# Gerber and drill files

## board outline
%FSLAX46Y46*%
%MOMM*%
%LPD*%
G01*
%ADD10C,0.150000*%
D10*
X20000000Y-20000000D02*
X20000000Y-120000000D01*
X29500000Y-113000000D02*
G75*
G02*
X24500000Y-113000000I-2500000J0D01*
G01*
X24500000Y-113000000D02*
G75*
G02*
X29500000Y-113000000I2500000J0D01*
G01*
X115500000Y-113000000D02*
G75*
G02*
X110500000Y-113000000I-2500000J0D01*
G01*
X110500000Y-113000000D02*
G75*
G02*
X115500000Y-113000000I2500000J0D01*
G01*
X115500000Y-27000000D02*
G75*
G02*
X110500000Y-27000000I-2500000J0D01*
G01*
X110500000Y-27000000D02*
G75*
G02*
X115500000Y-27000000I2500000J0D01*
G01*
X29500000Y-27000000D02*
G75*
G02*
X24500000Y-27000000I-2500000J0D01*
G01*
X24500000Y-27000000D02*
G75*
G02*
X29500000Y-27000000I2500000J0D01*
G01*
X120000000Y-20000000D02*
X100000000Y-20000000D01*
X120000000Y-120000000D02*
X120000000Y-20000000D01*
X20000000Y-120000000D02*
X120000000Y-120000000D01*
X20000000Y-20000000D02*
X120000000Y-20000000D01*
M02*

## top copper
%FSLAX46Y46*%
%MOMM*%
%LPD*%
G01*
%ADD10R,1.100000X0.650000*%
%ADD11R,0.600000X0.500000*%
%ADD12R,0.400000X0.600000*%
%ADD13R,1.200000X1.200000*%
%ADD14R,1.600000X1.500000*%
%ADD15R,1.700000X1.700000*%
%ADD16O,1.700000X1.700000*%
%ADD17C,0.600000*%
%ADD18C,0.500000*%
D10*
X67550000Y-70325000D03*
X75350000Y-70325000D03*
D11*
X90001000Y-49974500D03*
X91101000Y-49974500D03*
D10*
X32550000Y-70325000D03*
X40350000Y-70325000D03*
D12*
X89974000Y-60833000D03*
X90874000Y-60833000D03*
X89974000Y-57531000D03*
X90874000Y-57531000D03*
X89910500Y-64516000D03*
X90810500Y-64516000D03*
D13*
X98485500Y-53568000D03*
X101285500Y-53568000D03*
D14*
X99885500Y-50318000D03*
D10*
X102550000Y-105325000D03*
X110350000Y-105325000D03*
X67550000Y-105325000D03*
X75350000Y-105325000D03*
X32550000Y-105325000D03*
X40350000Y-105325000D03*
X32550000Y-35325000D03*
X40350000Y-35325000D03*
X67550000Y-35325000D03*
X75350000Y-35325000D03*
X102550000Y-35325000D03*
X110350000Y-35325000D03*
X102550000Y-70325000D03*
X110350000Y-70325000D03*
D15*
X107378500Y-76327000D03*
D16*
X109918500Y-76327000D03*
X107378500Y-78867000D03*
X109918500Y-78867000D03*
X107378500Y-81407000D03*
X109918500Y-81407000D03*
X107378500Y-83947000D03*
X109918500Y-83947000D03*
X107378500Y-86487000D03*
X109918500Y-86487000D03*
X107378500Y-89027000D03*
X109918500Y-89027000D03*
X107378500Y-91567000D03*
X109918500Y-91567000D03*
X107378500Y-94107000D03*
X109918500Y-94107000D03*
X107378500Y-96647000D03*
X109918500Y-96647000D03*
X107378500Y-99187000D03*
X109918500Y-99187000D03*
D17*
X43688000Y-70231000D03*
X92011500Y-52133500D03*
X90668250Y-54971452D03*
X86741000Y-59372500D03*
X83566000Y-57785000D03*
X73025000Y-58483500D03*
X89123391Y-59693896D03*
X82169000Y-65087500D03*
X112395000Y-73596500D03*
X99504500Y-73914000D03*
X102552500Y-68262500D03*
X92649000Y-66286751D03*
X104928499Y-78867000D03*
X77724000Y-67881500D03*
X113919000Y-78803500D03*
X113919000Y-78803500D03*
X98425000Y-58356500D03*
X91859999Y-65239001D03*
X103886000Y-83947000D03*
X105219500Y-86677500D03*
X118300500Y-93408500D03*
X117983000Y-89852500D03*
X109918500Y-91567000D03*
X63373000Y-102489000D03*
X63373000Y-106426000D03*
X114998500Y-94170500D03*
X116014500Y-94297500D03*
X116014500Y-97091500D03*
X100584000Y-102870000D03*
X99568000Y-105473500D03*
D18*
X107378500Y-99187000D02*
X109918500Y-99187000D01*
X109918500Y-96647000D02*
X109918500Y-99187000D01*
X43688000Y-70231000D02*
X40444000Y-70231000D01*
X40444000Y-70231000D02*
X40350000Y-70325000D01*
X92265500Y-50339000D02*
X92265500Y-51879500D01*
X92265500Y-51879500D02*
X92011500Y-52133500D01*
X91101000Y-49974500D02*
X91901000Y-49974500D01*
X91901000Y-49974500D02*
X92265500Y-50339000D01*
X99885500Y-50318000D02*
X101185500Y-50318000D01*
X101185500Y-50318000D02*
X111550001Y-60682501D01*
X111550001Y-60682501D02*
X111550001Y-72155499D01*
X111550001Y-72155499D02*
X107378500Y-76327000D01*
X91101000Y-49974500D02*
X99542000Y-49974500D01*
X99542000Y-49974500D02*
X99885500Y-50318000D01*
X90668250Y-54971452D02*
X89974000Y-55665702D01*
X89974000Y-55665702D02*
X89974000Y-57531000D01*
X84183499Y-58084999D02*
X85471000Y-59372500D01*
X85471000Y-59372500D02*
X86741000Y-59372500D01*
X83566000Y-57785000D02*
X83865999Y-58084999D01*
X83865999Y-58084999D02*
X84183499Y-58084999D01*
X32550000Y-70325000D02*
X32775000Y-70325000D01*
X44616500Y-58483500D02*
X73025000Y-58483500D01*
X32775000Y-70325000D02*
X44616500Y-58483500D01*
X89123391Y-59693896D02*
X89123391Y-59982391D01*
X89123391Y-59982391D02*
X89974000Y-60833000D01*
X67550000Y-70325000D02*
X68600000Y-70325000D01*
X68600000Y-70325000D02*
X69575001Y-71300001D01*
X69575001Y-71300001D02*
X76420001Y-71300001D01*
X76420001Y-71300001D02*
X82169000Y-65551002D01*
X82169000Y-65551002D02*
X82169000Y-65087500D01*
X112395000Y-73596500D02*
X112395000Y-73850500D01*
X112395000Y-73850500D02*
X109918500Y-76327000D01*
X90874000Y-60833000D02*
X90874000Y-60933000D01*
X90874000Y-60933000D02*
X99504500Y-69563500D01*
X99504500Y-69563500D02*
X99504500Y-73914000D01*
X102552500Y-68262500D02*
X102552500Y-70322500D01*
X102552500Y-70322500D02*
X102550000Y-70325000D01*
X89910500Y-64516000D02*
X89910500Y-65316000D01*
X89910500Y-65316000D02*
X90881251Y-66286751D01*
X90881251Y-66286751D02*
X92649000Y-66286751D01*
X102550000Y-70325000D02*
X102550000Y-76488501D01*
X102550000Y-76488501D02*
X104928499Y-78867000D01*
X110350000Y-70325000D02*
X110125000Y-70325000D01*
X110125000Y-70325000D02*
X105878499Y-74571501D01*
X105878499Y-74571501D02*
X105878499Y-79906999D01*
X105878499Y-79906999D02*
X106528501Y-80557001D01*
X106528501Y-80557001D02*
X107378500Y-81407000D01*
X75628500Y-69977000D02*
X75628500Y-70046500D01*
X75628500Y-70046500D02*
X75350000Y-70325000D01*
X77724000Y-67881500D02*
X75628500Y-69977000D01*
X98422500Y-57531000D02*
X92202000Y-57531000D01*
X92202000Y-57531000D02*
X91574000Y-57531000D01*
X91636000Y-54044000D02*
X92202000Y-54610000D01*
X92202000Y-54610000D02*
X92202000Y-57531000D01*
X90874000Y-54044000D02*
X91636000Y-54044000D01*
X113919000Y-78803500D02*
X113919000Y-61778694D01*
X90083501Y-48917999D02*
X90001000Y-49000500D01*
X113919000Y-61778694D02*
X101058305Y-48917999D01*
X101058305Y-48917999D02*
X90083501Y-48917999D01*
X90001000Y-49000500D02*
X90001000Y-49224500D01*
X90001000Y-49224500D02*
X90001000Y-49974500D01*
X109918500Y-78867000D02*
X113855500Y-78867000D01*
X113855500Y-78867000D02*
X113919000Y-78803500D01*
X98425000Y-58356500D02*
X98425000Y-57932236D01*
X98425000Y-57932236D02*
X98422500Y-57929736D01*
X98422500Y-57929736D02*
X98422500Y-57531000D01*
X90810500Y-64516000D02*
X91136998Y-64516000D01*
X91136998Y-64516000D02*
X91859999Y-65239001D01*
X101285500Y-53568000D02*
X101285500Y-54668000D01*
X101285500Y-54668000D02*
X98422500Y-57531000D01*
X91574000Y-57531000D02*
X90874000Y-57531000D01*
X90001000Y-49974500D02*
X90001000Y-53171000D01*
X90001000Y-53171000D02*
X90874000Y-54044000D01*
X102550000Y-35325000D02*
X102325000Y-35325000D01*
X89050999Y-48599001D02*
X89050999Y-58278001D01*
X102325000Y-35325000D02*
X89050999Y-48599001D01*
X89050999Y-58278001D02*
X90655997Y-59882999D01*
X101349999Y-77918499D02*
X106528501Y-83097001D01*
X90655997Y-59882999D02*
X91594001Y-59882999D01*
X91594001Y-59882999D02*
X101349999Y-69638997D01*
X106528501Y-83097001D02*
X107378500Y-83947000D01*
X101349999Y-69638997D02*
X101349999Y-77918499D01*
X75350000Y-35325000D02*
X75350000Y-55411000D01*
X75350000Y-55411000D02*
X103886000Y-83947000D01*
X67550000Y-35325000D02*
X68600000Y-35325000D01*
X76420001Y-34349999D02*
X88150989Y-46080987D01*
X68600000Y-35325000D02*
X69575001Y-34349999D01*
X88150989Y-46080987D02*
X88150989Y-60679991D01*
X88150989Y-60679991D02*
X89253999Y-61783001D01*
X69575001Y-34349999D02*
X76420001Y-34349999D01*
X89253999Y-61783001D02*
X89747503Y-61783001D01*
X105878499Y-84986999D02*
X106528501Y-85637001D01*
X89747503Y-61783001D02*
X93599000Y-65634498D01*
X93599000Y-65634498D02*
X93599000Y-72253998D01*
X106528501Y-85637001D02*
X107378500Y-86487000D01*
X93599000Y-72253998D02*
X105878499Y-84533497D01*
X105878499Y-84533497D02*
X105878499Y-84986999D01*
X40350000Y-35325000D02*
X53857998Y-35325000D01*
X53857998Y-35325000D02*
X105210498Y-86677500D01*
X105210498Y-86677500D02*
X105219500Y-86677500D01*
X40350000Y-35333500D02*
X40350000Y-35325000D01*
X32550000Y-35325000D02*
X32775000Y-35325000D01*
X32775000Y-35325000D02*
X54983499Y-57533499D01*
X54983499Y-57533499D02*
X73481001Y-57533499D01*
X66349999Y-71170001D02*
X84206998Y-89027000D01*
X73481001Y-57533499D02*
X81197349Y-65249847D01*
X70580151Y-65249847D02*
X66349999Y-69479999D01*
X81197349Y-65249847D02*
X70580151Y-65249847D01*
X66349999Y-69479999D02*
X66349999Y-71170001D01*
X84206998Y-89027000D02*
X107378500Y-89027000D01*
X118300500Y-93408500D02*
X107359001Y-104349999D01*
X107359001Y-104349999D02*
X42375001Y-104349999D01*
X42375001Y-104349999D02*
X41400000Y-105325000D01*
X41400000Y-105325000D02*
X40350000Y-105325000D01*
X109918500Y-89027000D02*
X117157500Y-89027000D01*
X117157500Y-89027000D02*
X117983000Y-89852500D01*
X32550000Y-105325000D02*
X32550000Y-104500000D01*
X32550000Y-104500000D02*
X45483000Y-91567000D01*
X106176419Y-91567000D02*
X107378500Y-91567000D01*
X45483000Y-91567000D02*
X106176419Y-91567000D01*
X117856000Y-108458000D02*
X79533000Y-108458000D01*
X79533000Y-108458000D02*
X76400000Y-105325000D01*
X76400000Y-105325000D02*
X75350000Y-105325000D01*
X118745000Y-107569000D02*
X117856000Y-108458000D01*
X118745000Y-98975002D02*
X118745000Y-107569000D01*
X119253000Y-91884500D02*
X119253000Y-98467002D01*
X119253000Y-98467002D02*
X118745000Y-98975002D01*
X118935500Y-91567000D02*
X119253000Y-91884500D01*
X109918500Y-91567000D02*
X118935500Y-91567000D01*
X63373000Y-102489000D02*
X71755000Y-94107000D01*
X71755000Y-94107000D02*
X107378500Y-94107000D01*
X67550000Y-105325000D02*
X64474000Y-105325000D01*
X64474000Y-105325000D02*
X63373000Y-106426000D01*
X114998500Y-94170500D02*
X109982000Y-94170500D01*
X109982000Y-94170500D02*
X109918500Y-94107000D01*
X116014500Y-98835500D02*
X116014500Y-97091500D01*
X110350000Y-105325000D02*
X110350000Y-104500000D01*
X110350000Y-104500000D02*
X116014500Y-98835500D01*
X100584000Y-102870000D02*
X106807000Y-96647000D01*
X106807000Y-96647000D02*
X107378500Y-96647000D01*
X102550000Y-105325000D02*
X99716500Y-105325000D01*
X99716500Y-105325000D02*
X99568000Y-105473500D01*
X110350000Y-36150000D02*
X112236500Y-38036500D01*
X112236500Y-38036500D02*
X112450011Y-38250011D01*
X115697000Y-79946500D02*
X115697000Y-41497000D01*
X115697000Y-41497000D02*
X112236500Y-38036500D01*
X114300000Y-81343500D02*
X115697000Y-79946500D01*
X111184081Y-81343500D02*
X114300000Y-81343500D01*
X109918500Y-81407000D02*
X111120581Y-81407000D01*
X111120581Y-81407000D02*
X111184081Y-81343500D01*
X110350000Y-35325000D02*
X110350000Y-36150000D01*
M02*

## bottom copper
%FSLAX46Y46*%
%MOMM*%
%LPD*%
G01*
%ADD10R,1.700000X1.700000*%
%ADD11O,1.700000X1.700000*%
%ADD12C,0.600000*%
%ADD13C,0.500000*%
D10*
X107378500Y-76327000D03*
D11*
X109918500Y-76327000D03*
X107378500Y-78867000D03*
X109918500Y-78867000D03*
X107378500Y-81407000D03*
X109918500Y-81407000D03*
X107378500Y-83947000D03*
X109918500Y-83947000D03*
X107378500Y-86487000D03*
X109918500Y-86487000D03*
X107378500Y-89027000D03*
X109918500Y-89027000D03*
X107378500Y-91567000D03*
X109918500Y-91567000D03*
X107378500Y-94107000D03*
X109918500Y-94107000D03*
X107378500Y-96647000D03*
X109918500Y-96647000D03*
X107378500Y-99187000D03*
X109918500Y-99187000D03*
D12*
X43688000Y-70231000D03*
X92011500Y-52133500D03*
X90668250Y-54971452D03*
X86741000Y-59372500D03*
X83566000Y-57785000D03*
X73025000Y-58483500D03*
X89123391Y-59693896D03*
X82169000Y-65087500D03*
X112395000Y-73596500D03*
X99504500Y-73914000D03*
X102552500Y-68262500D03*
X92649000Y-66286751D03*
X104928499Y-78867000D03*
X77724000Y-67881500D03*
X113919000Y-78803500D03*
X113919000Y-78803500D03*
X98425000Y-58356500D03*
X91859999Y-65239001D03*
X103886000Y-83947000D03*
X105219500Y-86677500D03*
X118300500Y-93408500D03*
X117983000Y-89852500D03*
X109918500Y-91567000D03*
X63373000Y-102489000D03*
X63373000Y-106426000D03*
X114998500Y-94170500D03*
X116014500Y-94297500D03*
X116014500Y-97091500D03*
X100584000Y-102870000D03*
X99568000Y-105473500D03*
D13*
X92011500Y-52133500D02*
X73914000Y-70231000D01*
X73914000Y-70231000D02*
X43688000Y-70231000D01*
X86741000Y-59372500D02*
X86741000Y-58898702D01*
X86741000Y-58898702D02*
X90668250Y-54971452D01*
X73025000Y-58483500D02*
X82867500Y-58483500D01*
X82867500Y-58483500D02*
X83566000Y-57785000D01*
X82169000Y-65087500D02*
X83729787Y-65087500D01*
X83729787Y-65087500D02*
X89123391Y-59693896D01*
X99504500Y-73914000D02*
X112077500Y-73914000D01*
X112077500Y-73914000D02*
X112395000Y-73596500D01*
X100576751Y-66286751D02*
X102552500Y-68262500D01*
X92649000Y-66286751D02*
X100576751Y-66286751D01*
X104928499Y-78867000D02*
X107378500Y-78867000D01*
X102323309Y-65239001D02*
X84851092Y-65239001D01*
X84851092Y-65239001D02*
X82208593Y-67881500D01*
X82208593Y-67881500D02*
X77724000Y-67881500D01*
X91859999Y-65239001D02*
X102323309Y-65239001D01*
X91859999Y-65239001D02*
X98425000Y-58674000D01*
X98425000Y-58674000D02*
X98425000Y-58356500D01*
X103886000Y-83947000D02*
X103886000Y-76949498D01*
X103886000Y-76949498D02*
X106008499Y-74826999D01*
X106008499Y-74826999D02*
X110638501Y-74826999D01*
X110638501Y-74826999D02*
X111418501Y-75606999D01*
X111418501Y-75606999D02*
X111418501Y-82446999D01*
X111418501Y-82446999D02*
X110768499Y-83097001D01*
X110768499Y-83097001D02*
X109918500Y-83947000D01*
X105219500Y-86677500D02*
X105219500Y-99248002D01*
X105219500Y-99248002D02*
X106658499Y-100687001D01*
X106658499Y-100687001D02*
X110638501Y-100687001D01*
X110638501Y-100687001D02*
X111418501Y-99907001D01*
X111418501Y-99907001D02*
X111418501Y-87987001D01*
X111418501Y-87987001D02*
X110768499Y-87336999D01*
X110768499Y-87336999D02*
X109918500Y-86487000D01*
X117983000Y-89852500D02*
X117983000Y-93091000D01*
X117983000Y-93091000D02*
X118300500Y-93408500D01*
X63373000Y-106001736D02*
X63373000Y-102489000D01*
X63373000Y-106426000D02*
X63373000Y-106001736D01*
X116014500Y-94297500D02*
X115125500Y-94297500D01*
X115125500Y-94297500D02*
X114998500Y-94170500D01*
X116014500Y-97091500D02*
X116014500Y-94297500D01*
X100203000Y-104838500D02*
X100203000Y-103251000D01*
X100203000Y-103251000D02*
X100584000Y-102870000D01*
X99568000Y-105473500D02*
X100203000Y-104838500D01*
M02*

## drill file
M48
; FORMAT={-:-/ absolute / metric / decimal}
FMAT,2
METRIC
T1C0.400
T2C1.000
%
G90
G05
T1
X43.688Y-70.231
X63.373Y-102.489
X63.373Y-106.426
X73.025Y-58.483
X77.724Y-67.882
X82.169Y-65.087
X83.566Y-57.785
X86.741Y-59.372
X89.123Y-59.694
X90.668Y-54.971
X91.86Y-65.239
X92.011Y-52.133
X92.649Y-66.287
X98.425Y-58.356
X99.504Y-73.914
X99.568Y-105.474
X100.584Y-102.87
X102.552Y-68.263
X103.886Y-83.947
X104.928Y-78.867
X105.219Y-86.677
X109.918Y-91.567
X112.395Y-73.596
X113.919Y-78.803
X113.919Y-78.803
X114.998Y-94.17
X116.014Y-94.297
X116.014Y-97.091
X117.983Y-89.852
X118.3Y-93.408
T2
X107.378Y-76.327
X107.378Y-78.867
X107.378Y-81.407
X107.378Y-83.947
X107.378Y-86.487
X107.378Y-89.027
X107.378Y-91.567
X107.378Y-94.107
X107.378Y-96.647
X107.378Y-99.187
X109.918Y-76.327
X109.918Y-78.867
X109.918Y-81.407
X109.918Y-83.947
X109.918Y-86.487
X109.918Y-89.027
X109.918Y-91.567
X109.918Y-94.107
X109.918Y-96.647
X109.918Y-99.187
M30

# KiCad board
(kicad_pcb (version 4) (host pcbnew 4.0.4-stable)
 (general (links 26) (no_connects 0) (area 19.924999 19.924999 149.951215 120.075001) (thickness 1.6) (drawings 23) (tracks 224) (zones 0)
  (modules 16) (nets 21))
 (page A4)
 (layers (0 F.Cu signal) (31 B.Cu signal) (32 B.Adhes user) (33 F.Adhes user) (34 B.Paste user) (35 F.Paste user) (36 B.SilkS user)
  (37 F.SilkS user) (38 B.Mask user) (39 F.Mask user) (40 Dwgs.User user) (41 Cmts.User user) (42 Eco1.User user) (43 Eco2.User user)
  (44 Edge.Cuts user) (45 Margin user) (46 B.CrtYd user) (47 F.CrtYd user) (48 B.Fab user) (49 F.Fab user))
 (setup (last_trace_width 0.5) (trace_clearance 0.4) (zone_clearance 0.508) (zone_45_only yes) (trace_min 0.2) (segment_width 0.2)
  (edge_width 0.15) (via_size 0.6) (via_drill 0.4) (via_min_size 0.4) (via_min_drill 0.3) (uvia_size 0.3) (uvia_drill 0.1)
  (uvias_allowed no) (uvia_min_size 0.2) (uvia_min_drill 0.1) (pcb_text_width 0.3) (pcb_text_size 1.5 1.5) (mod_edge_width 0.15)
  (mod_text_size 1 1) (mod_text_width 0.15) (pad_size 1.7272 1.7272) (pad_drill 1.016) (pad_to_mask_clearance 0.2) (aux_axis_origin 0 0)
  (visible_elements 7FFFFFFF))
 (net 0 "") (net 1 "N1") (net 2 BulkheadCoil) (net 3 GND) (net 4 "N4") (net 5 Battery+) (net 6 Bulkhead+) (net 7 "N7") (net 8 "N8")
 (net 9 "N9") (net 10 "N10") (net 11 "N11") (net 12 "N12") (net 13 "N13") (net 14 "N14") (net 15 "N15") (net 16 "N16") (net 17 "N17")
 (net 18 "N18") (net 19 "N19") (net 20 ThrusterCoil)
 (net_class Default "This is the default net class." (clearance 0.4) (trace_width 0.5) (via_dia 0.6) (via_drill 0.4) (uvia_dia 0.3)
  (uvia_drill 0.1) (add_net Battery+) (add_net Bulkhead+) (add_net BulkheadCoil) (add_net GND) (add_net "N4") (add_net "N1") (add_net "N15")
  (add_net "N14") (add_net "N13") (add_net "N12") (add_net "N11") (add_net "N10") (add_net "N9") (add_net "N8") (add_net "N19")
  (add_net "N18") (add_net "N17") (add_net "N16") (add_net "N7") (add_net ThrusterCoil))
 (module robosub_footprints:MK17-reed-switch (layer F.Cu) (at 67 70)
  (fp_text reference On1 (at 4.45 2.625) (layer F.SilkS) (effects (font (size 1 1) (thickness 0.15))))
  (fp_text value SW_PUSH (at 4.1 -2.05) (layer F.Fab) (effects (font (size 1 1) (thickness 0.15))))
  (pad 1 smd rect (at 0.55 0.325) (size 1.1 0.65) (layers F.Cu F.Paste F.Mask) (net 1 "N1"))
  (pad 2 smd rect (at 8.35 0.325) (size 1.1 0.65) (layers F.Cu F.Paste F.Mask) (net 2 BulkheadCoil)))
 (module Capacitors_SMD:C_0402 (layer F.Cu) (at 90.551 49.9745)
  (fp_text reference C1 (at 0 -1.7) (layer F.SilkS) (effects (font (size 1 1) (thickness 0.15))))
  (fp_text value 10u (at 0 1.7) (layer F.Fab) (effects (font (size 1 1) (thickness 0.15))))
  (pad 1 smd rect (at -0.55 0) (size 0.6 0.5) (layers F.Cu F.Paste F.Mask) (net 2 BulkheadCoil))
  (pad 2 smd rect (at 0.55 0) (size 0.6 0.5) (layers F.Cu F.Paste F.Mask) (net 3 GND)))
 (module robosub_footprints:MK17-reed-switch (layer F.Cu) (at 32 70)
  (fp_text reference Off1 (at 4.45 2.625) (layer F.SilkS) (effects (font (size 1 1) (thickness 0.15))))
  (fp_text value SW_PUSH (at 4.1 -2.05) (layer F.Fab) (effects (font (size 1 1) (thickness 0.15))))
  (pad 1 smd rect (at 0.55 0.325) (size 1.1 0.65) (layers F.Cu F.Paste F.Mask) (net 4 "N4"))
  (pad 2 smd rect (at 8.35 0.325) (size 1.1 0.65) (layers F.Cu F.Paste F.Mask) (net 3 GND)))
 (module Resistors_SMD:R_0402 (layer F.Cu) (at 90.424 60.833)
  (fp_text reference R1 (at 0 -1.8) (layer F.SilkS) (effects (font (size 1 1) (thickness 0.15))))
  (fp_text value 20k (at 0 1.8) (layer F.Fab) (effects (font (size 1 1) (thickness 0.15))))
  (pad 1 smd rect (at -0.45 0) (size 0.4 0.6) (layers F.Cu F.Paste F.Mask) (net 1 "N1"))
  (pad 2 smd rect (at 0.45 0) (size 0.4 0.6) (layers F.Cu F.Paste F.Mask) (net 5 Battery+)))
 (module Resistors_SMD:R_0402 (layer F.Cu) (at 90.424 57.531)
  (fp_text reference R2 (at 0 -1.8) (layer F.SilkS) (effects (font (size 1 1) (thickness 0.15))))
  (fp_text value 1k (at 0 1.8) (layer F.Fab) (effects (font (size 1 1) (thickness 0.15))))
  (pad 1 smd rect (at -0.45 0) (size 0.4 0.6) (layers F.Cu F.Paste F.Mask) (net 4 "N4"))
  (pad 2 smd rect (at 0.45 0) (size 0.4 0.6) (layers F.Cu F.Paste F.Mask) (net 2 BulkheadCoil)))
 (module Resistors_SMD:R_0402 (layer F.Cu) (at 90.3605 64.516)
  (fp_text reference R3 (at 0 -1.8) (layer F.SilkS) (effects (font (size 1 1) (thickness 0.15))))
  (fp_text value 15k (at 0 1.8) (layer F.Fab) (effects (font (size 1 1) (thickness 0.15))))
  (pad 1 smd rect (at -0.45 0) (size 0.4 0.6) (layers F.Cu F.Paste F.Mask) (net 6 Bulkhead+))
  (pad 2 smd rect (at 0.45 0) (size 0.4 0.6) (layers F.Cu F.Paste F.Mask) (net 2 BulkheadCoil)))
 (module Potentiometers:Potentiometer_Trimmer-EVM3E (layer F.Cu) (at 99.8855 51.943)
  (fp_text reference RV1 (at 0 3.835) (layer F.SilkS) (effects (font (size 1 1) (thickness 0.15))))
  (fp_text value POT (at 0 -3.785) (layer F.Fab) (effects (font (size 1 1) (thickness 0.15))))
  (pad 1 smd rect (at -1.4 1.625) (size 1.2 1.2) (layers F.Cu F.Paste F.Mask) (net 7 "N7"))
  (pad 3 smd rect (at 1.4 1.625) (size 1.2 1.2) (layers F.Cu F.Paste F.Mask) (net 2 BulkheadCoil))
  (pad 2 smd rect (at 0 -1.625) (size 1.6 1.5) (layers F.Cu F.Paste F.Mask) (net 3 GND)))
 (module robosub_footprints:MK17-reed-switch (layer F.Cu) (at 102 105)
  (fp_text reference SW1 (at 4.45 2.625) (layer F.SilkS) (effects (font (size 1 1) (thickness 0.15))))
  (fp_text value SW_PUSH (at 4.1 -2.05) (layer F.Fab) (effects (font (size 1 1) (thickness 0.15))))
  (pad 1 smd rect (at 0.55 0.325) (size 1.1 0.65) (layers F.Cu F.Paste F.Mask) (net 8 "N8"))
  (pad 2 smd rect (at 8.35 0.325) (size 1.1 0.65) (layers F.Cu F.Paste F.Mask) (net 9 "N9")))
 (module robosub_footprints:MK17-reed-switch (layer F.Cu) (at 67 105)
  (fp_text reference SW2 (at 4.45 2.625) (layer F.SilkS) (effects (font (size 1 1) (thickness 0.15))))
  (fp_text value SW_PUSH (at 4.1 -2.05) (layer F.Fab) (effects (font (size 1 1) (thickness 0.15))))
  (pad 1 smd rect (at 0.55 0.325) (size 1.1 0.65) (layers F.Cu F.Paste F.Mask) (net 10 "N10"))
  (pad 2 smd rect (at 8.35 0.325) (size 1.1 0.65) (layers F.Cu F.Paste F.Mask) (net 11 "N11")))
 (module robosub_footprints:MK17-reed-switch (layer F.Cu) (at 32 105)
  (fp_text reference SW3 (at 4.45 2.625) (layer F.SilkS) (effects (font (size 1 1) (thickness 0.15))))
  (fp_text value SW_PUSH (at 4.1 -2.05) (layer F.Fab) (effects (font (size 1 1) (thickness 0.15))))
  (pad 1 smd rect (at 0.55 0.325) (size 1.1 0.65) (layers F.Cu F.Paste F.Mask) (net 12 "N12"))
  (pad 2 smd rect (at 8.35 0.325) (size 1.1 0.65) (layers F.Cu F.Paste F.Mask) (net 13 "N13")))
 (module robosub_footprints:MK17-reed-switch (layer F.Cu) (at 32 35)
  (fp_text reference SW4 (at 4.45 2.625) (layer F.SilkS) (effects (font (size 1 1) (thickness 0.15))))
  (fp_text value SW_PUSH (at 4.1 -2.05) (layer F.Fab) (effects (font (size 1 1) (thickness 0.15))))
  (pad 1 smd rect (at 0.55 0.325) (size 1.1 0.65) (layers F.Cu F.Paste F.Mask) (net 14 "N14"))
  (pad 2 smd rect (at 8.35 0.325) (size 1.1 0.65) (layers F.Cu F.Paste F.Mask) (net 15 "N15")))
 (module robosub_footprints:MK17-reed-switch (layer F.Cu) (at 67 35)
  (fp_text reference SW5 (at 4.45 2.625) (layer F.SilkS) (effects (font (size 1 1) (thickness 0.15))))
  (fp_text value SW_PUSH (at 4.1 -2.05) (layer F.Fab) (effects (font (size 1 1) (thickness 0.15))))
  (pad 1 smd rect (at 0.55 0.325) (size 1.1 0.65) (layers F.Cu F.Paste F.Mask) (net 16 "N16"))
  (pad 2 smd rect (at 8.35 0.325) (size 1.1 0.65) (layers F.Cu F.Paste F.Mask) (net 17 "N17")))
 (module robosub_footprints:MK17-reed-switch (layer F.Cu) (at 102 35)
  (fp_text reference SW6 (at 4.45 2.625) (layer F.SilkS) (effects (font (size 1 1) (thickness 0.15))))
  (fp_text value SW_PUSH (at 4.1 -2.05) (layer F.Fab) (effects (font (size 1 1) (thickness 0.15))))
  (pad 1 smd rect (at 0.55 0.325) (size 1.1 0.65) (layers F.Cu F.Paste F.Mask) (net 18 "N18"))
  (pad 2 smd rect (at 8.35 0.325) (size 1.1 0.65) (layers F.Cu F.Paste F.Mask) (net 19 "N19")))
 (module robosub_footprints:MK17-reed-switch (layer F.Cu) (at 102 70)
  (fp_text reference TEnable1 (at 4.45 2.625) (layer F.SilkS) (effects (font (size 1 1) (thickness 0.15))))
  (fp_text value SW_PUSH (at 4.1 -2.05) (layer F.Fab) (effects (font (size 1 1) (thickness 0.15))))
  (pad 1 smd rect (at 0.55 0.325) (size 1.1 0.65) (layers F.Cu F.Paste F.Mask) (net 6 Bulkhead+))
  (pad 2 smd rect (at 8.35 0.325) (size 1.1 0.65) (layers F.Cu F.Paste F.Mask) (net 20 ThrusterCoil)))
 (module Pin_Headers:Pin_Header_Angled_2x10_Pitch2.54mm (layer F.Cu) (at 107.3785 76.327)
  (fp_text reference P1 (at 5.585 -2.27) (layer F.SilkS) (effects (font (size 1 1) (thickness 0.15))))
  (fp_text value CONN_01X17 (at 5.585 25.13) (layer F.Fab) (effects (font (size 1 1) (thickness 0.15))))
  (pad 1 thru_hole rect (at 0 0) (size 1.7 1.7) (drill 1) (layers *.Cu *.Mask) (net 3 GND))
  (pad 2 thru_hole oval (at 2.54 0) (size 1.7 1.7) (drill 1) (layers *.Cu *.Mask) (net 5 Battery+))
  (pad 3 thru_hole oval (at 0 2.54) (size 1.7 1.7) (drill 1) (layers *.Cu *.Mask) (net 6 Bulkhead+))
  (pad 4 thru_hole oval (at 2.54 2.54) (size 1.7 1.7) (drill 1) (layers *.Cu *.Mask) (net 2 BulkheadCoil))
  (pad 5 thru_hole oval (at 0 5.08) (size 1.7 1.7) (drill 1) (layers *.Cu *.Mask) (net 20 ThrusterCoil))
  (pad 6 thru_hole oval (at 2.54 5.08) (size 1.7 1.7) (drill 1) (layers *.Cu *.Mask) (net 19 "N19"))
  (pad 7 thru_hole oval (at 0 7.62) (size 1.7 1.7) (drill 1) (layers *.Cu *.Mask) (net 18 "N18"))
  (pad 8 thru_hole oval (at 2.54 7.62) (size 1.7 1.7) (drill 1) (layers *.Cu *.Mask) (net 17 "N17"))
  (pad 9 thru_hole oval (at 0 10.16) (size 1.7 1.7) (drill 1) (layers *.Cu *.Mask) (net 16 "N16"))
  (pad 10 thru_hole oval (at 2.54 10.16) (size 1.7 1.7) (drill 1) (layers *.Cu *.Mask) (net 15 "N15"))
  (pad 11 thru_hole oval (at 0 12.7) (size 1.7 1.7) (drill 1) (layers *.Cu *.Mask) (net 14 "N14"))
  (pad 12 thru_hole oval (at 2.54 12.7) (size 1.7 1.7) (drill 1) (layers *.Cu *.Mask) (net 13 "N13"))
  (pad 13 thru_hole oval (at 0 15.24) (size 1.7 1.7) (drill 1) (layers *.Cu *.Mask) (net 12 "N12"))
  (pad 14 thru_hole oval (at 2.54 15.24) (size 1.7 1.7) (drill 1) (layers *.Cu *.Mask) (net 11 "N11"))
  (pad 15 thru_hole oval (at 0 17.78) (size 1.7 1.7) (drill 1) (layers *.Cu *.Mask) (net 10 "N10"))
  (pad 16 thru_hole oval (at 2.54 17.78) (size 1.7 1.7) (drill 1) (layers *.Cu *.Mask) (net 9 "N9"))
  (pad 17 thru_hole oval (at 0 20.32) (size 1.7 1.7) (drill 1) (layers *.Cu *.Mask) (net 8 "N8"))
  (pad 18 thru_hole oval (at 2.54 20.32) (size 1.7 1.7) (drill 1) (layers *.Cu *.Mask))
  (pad 19 thru_hole oval (at 0 22.86) (size 1.7 1.7) (drill 1) (layers *.Cu *.Mask))
  (pad 20 thru_hole oval (at 2.54 22.86) (size 1.7 1.7) (drill 1) (layers *.Cu *.Mask)))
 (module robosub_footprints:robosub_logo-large (layer F.Cu) (at 49.403 79.5655)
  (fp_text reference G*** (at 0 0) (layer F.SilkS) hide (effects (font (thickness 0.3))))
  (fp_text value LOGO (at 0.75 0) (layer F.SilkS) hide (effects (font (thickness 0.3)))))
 (gr_line (start 20 20) (end 20 120) (angle 90) (layer Edge.Cuts) (width 0.15))
 (gr_circle (center 27 113) (end 24.5 113) (layer Edge.Cuts) (width 0.15))
 (gr_circle (center 113 113) (end 115.5 113) (layer Edge.Cuts) (width 0.15))
 (gr_circle (center 113 27) (end 115.5 27) (layer Edge.Cuts) (width 0.15))
 (gr_circle (center 27 27) (end 24.5 27) (layer Edge.Cuts) (width 0.15))
 (gr_line (start 120 20) (end 100 20) (angle 90) (layer Edge.Cuts) (width 0.15))
 (gr_line (start 120 120) (end 120 20) (angle 90) (layer Edge.Cuts) (width 0.15))
 (gr_line (start 20 120) (end 120 120) (angle 90) (layer Edge.Cuts) (width 0.15))
 (gr_line (start 20 20) (end 120 20) (angle 90) (layer Edge.Cuts) (width 0.15))
 (segment (start 107.3785 99.187) (end 109.9185 99.187) (width 0.5) (layer F.Cu) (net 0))
 (segment (start 109.9185 96.647) (end 109.9185 99.187) (width 0.5) (layer F.Cu) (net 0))
 (segment (start 43.688 70.231) (end 40.444 70.231) (width 0.5) (layer F.Cu) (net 3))
 (segment (start 40.444 70.231) (end 40.35 70.325) (width 0.5) (layer F.Cu) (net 3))
 (segment (start 92.0115 52.1335) (end 73.914 70.231) (width 0.5) (layer B.Cu) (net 3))
 (segment (start 73.914 70.231) (end 43.688 70.231) (width 0.5) (layer B.Cu) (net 3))
 (via (at 43.688 70.231) (size 0.6) (drill 0.4) (layers F.Cu B.Cu) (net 3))
 (segment (start 92.2655 50.339) (end 92.2655 51.8795) (width 0.5) (layer F.Cu) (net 3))
 (segment (start 92.2655 51.8795) (end 92.0115 52.1335) (width 0.5) (layer F.Cu) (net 3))
 (via (at 92.0115 52.1335) (size 0.6) (drill 0.4) (layers F.Cu B.Cu) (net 3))
 (segment (start 91.101 49.9745) (end 91.901 49.9745) (width 0.5) (layer F.Cu) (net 3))
 (segment (start 91.901 49.9745) (end 92.2655 50.339) (width 0.5) (layer F.Cu) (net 3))
 (segment (start 99.8855 50.318) (end 101.1855 50.318) (width 0.5) (layer F.Cu) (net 3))
 (segment (start 101.1855 50.318) (end 111.550001 60.682501) (width 0.5) (layer F.Cu) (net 3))
 (segment (start 111.550001 60.682501) (end 111.550001 72.155499) (width 0.5) (layer F.Cu) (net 3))
 (segment (start 111.550001 72.155499) (end 107.3785 76.327) (width 0.5) (layer F.Cu) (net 3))
 (segment (start 91.101 49.9745) (end 99.542 49.9745) (width 0.5) (layer F.Cu) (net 3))
 (segment (start 99.542 49.9745) (end 99.8855 50.318) (width 0.5) (layer F.Cu) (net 3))
 (segment (start 90.66825 54.971452) (end 89.974 55.665702) (width 0.5) (layer F.Cu) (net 4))
 (segment (start 89.974 55.665702) (end 89.974 57.531) (width 0.5) (layer F.Cu) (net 4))
 (segment (start 86.741 59.3725) (end 86.741 58.898702) (width 0.5) (layer B.Cu) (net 4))
 (via (at 90.66825 54.971452) (size 0.6) (drill 0.4) (layers F.Cu B.Cu) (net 4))
 (segment (start 86.741 58.898702) (end 90.66825 54.971452) (width 0.5) (layer B.Cu) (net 4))
 (segment (start 84.183499 58.084999) (end 85.471 59.3725) (width 0.5) (layer F.Cu) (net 4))
 (segment (start 85.471 59.3725) (end 86.741 59.3725) (width 0.5) (layer F.Cu) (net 4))
 (via (at 86.741 59.3725) (size 0.6) (drill 0.4) (layers F.Cu B.Cu) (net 4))
 (segment (start 83.566 57.785) (end 83.865999 58.084999) (width 0.5) (layer F.Cu) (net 4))
 (segment (start 83.865999 58.084999) (end 84.183499 58.084999) (width 0.5) (layer F.Cu) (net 4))
 (segment (start 73.025 58.4835) (end 82.8675 58.4835) (width 0.5) (layer B.Cu) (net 4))
 (segment (start 82.8675 58.4835) (end 83.566 57.785) (width 0.5) (layer B.Cu) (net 4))
 (via (at 83.566 57.785) (size 0.6) (drill 0.4) (layers F.Cu B.Cu) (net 4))
 (segment (start 32.55 70.325) (end 32.775 70.325) (width 0.5) (layer F.Cu) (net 4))
 (segment (start 44.6165 58.4835) (end 73.025 58.4835) (width 0.5) (layer F.Cu) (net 4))
 (segment (start 32.775 70.325) (end 44.6165 58.4835) (width 0.5) (layer F.Cu) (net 4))
 (via (at 73.025 58.4835) (size 0.6) (drill 0.4) (layers F.Cu B.Cu) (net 4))
 (segment (start 89.123391 59.693896) (end 89.123391 59.982391) (width 0.5) (layer F.Cu) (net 1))
 (segment (start 89.123391 59.982391) (end 89.974 60.833) (width 0.5) (layer F.Cu) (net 1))
 (segment (start 82.169 65.0875) (end 83.729787 65.0875) (width 0.5) (layer B.Cu) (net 1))
 (segment (start 83.729787 65.0875) (end 89.123391 59.693896) (width 0.5) (layer B.Cu) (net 1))
 (via (at 89.123391 59.693896) (size 0.6) (drill 0.4) (layers F.Cu B.Cu) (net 1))
 (segment (start 67.55 70.325) (end 68.6 70.325) (width 0.5) (layer F.Cu) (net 1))
 (segment (start 68.6 70.325) (end 69.575001 71.300001) (width 0.5) (layer F.Cu) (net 1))
 (segment (start 69.575001 71.300001) (end 76.420001 71.300001) (width 0.5) (layer F.Cu) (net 1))
 (via (at 82.169 65.0875) (size 0.6) (drill 0.4) (layers F.Cu B.Cu) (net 1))
 (segment (start 76.420001 71.300001) (end 82.169 65.551002) (width 0.5) (layer F.Cu) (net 1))
 (segment (start 82.169 65.551002) (end 82.169 65.0875) (width 0.5) (layer F.Cu) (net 1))
 (segment (start 112.395 73.5965) (end 112.395 73.8505) (width 0.5) (layer F.Cu) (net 5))
 (segment (start 112.395 73.8505) (end 109.9185 76.327) (width 0.5) (layer F.Cu) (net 5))
 (segment (start 99.5045 73.914) (end 112.0775 73.914) (width 0.5) (layer B.Cu) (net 5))
 (segment (start 112.0775 73.914) (end 112.395 73.5965) (width 0.5) (layer B.Cu) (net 5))
 (via (at 112.395 73.5965) (size 0.6) (drill 0.4) (layers F.Cu B.Cu) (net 5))
 (segment (start 90.874 60.833) (end 90.874 60.933) (width 0.5) (layer F.Cu) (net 5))
 (segment (start 90.874 60.933) (end 99.5045 69.5635) (width 0.5) (layer F.Cu) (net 5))
 (segment (start 99.5045 69.5635) (end 99.5045 73.914) (width 0.5) (layer F.Cu) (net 5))
 (via (at 99.5045 73.914) (size 0.6) (drill 0.4) (layers F.Cu B.Cu) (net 5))
 (segment (start 102.5525 68.2625) (end 102.5525 70.3225) (width 0.5) (layer F.Cu) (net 6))
 (segment (start 102.5525 70.3225) (end 102.55 70.325) (width 0.5) (layer F.Cu) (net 6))
 (segment (start 100.576751 66.286751) (end 102.5525 68.2625) (width 0.5) (layer B.Cu) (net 6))
 (via (at 102.5525 68.2625) (size 0.6) (drill 0.4) (layers F.Cu B.Cu) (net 6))
 (segment (start 92.649 66.286751) (end 100.576751 66.286751) (width 0.5) (layer B.Cu) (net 6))
 (segment (start 89.9105 64.516) (end 89.9105 65.316) (width 0.5) (layer F.Cu) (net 6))
 (segment (start 89.9105 65.316) (end 90.881251 66.286751) (width 0.5) (layer F.Cu) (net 6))
 (segment (start 90.881251 66.286751) (end 92.649 66.286751) (width 0.5) (layer F.Cu) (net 6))
 (via (at 92.649 66.286751) (size 0.6) (drill 0.4) (layers F.Cu B.Cu) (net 6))
 (segment (start 104.928499 78.867) (end 107.3785 78.867) (width 0.5) (layer B.Cu) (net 6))
 (segment (start 102.55 70.325) (end 102.55 76.488501) (width 0.5) (layer F.Cu) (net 6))
 (segment (start 102.55 76.488501) (end 104.928499 78.867) (width 0.5) (layer F.Cu) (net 6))
 (via (at 104.928499 78.867) (size 0.6) (drill 0.4) (layers F.Cu B.Cu) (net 6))
 (segment (start 110.35 70.325) (end 110.125 70.325) (width 0.5) (layer F.Cu) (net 20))
 (segment (start 110.125 70.325) (end 105.878499 74.571501) (width 0.5) (layer F.Cu) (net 20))
 (segment (start 105.878499 74.571501) (end 105.878499 79.906999) (width 0.5) (layer F.Cu) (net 20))
 (segment (start 105.878499 79.906999) (end 106.528501 80.557001) (width 0.5) (layer F.Cu) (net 20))
 (segment (start 106.528501 80.557001) (end 107.3785 81.407) (width 0.5) (layer F.Cu) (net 20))
 (segment (start 75.6285 69.977) (end 75.6285 70.0465) (width 0.5) (layer F.Cu) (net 2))
 (segment (start 75.6285 70.0465) (end 75.35 70.325) (width 0.5) (layer F.Cu) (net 2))
 (segment (start 77.724 67.8815) (end 75.6285 69.977) (width 0.5) (layer F.Cu) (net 2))
 (segment (start 102.323309 65.239001) (end 84.851092 65.239001) (width 0.5) (layer B.Cu) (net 2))
 (segment (start 84.851092 65.239001) (end 82.208593 67.8815) (width 0.5) (layer B.Cu) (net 2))
 (segment (start 82.208593 67.8815) (end 77.724 67.8815) (width 0.5) (layer B.Cu) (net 2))
 (via (at 77.724 67.8815) (size 0.6) (drill 0.4) (layers F.Cu B.Cu) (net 2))
 (segment (start 98.4225 57.531) (end 92.202 57.531) (width 0.5) (layer F.Cu) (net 2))
 (segment (start 92.202 57.531) (end 91.574 57.531) (width 0.5) (layer F.Cu) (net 2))
 (segment (start 91.636 54.044) (end 92.202 54.61) (width 0.5) (layer F.Cu) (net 2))
 (segment (start 92.202 54.61) (end 92.202 57.531) (width 0.5) (layer F.Cu) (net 2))
 (segment (start 90.874 54.044) (end 91.636 54.044) (width 0.5) (layer F.Cu) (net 2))
 (segment (start 113.919 78.8035) (end 113.919 61.778694) (width 0.5) (layer F.Cu) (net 2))
 (segment (start 90.083501 48.917999) (end 90.001 49.0005) (width 0.5) (layer F.Cu) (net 2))
 (segment (start 113.919 61.778694) (end 101.058305 48.917999) (width 0.5) (layer F.Cu) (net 2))
 (segment (start 101.058305 48.917999) (end 90.083501 48.917999) (width 0.5) (layer F.Cu) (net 2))
 (segment (start 90.001 49.0005) (end 90.001 49.2245) (width 0.5) (layer F.Cu) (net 2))
 (segment (start 90.001 49.2245) (end 90.001 49.9745) (width 0.5) (layer F.Cu) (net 2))
 (segment (start 109.9185 78.867) (end 113.8555 78.867) (width 0.5) (layer F.Cu) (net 2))
 (segment (start 113.8555 78.867) (end 113.919 78.8035) (width 0.5) (layer F.Cu) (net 2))
 (via (at 113.919 78.8035) (size 0.6) (drill 0.4) (layers F.Cu B.Cu) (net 2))
 (segment (start 91.859999 65.239001) (end 102.323309 65.239001) (width 0.5) (layer B.Cu) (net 2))
 (via (at 113.919 78.8035) (size 0.6) (drill 0.4) (layers F.Cu B.Cu) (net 2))
 (segment (start 98.425 58.3565) (end 98.425 57.932236) (width 0.5) (layer F.Cu) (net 2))
 (segment (start 98.425 57.932236) (end 98.4225 57.929736) (width 0.5) (layer F.Cu) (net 2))
 (segment (start 98.4225 57.929736) (end 98.4225 57.531) (width 0.5) (layer F.Cu) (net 2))
 (segment (start 91.859999 65.239001) (end 98.425 58.674) (width 0.5) (layer B.Cu) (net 2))
 (segment (start 98.425 58.674) (end 98.425 58.3565) (width 0.5) (layer B.Cu) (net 2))
 (via (at 98.425 58.3565) (size 0.6) (drill 0.4) (layers F.Cu B.Cu) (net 2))
 (segment (start 90.8105 64.516) (end 91.136998 64.516) (width 0.5) (layer F.Cu) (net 2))
 (via (at 91.859999 65.239001) (size 0.6) (drill 0.4) (layers F.Cu B.Cu) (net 2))
 (segment (start 91.136998 64.516) (end 91.859999 65.239001) (width 0.5) (layer F.Cu) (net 2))
 (segment (start 101.2855 53.568) (end 101.2855 54.668) (width 0.5) (layer F.Cu) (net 2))
 (segment (start 101.2855 54.668) (end 98.4225 57.531) (width 0.5) (layer F.Cu) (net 2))
 (segment (start 91.574 57.531) (end 90.874 57.531) (width 0.5) (layer F.Cu) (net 2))
 (segment (start 90.001 49.9745) (end 90.001 53.171) (width 0.5) (layer F.Cu) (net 2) (status 10))
 (segment (start 90.001 53.171) (end 90.874 54.044) (width 0.5) (layer F.Cu) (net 2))
 (segment (start 102.55 35.325) (end 102.325 35.325) (width 0.5) (layer F.Cu) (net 18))
 (segment (start 89.050999 48.599001) (end 89.050999 58.278001) (width 0.5) (layer F.Cu) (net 18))
 (segment (start 102.325 35.325) (end 89.050999 48.599001) (width 0.5) (layer F.Cu) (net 18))
 (segment (start 89.050999 58.278001) (end 90.655997 59.882999) (width 0.5) (layer F.Cu) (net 18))
 (segment (start 101.349999 77.918499) (end 106.528501 83.097001) (width 0.5) (layer F.Cu) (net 18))
 (segment (start 90.655997 59.882999) (end 91.594001 59.882999) (width 0.5) (layer F.Cu) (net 18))
 (segment (start 91.594001 59.882999) (end 101.349999 69.638997) (width 0.5) (layer F.Cu) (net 18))
 (segment (start 106.528501 83.097001) (end 107.3785 83.947) (width 0.5) (layer F.Cu) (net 18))
 (segment (start 101.349999 69.638997) (end 101.349999 77.918499) (width 0.5) (layer F.Cu) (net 18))
 (segment (start 103.886 83.947) (end 103.886 76.949498) (width 0.5) (layer B.Cu) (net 17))
 (segment (start 103.886 76.949498) (end 106.008499 74.826999) (width 0.5) (layer B.Cu) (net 17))
 (segment (start 106.008499 74.826999) (end 110.638501 74.826999) (width 0.5) (layer B.Cu) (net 17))
 (segment (start 110.638501 74.826999) (end 111.418501 75.606999) (width 0.5) (layer B.Cu) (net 17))
 (segment (start 111.418501 75.606999) (end 111.418501 82.446999) (width 0.5) (layer B.Cu) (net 17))
 (segment (start 111.418501 82.446999) (end 110.768499 83.097001) (width 0.5) (layer B.Cu) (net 17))
 (segment (start 110.768499 83.097001) (end 109.9185 83.947) (width 0.5) (layer B.Cu) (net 17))
 (segment (start 75.35 35.325) (end 75.35 55.411) (width 0.5) (layer F.Cu) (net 17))
 (segment (start 75.35 55.411) (end 103.886 83.947) (width 0.5) (layer F.Cu) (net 17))
 (via (at 103.886 83.947) (size 0.6) (drill 0.4) (layers F.Cu B.Cu) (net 17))
 (segment (start 67.55 35.325) (end 68.6 35.325) (width 0.5) (layer F.Cu) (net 16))
 (segment (start 76.420001 34.349999) (end 88.150989 46.080987) (width 0.5) (layer F.Cu) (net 16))
 (segment (start 68.6 35.325) (end 69.575001 34.349999) (width 0.5) (layer F.Cu) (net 16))
 (segment (start 88.150989 46.080987) (end 88.150989 60.679991) (width 0.5) (layer F.Cu) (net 16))
 (segment (start 88.150989 60.679991) (end 89.253999 61.783001) (width 0.5) (layer F.Cu) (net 16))
 (segment (start 69.575001 34.349999) (end 76.420001 34.349999) (width 0.5) (layer F.Cu) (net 16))
 (segment (start 89.253999 61.783001) (end 89.747503 61.783001) (width 0.5) (layer F.Cu) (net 16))
 (segment (start 105.878499 84.986999) (end 106.528501 85.637001) (width 0.5) (layer F.Cu) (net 16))
 (segment (start 89.747503 61.783001) (end 93.599 65.634498) (width 0.5) (layer F.Cu) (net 16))
 (segment (start 93.599 65.634498) (end 93.599 72.253998) (width 0.5) (layer F.Cu) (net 16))
 (segment (start 106.528501 85.637001) (end 107.3785 86.487) (width 0.5) (layer F.Cu) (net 16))
 (segment (start 93.599 72.253998) (end 105.878499 84.533497) (width 0.5) (layer F.Cu) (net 16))
 (segment (start 105.878499 84.533497) (end 105.878499 84.986999) (width 0.5) (layer F.Cu) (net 16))
 (segment (start 105.2195 86.6775) (end 105.2195 99.248002) (width 0.5) (layer B.Cu) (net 15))
 (segment (start 105.2195 99.248002) (end 106.658499 100.687001) (width 0.5) (layer B.Cu) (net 15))
 (segment (start 106.658499 100.687001) (end 110.638501 100.687001) (width 0.5) (layer B.Cu) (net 15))
 (segment (start 110.638501 100.687001) (end 111.418501 99.907001) (width 0.5) (layer B.Cu) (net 15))
 (segment (start 111.418501 99.907001) (end 111.418501 87.987001) (width 0.5) (layer B.Cu) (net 15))
 (segment (start 111.418501 87.987001) (end 110.768499 87.336999) (width 0.5) (layer B.Cu) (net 15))
 (segment (start 110.768499 87.336999) (end 109.9185 86.487) (width 0.5) (layer B.Cu) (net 15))
 (segment (start 40.35 35.325) (end 53.857998 35.325) (width 0.5) (layer F.Cu) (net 15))
 (segment (start 53.857998 35.325) (end 105.210498 86.6775) (width 0.5) (layer F.Cu) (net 15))
 (segment (start 105.210498 86.6775) (end 105.2195 86.6775) (width 0.5) (layer F.Cu) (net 15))
 (via (at 105.2195 86.6775) (size 0.6) (drill 0.4) (layers F.Cu B.Cu) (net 15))
 (segment (start 40.35 35.3335) (end 40.35 35.325) (width 0.5) (layer F.Cu) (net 15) (status 30))
 (segment (start 32.55 35.325) (end 32.775 35.325) (width 0.5) (layer F.Cu) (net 14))
 (segment (start 32.775 35.325) (end 54.983499 57.533499) (width 0.5) (layer F.Cu) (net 14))
 (segment (start 54.983499 57.533499) (end 73.481001 57.533499) (width 0.5) (layer F.Cu) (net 14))
 (segment (start 66.349999 71.170001) (end 84.206998 89.027) (width 0.5) (layer F.Cu) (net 14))
 (segment (start 73.481001 57.533499) (end 81.197349 65.249847) (width 0.5) (layer F.Cu) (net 14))
 (segment (start 70.580151 65.249847) (end 66.349999 69.479999) (width 0.5) (layer F.Cu) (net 14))
 (segment (start 81.197349 65.249847) (end 70.580151 65.249847) (width 0.5) (layer F.Cu) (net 14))
 (segment (start 66.349999 69.479999) (end 66.349999 71.170001) (width 0.5) (layer F.Cu) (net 14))
 (segment (start 84.206998 89.027) (end 107.3785 89.027) (width 0.5) (layer F.Cu) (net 14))
 (segment (start 118.3005 93.4085) (end 107.359001 104.349999) (width 0.5) (layer F.Cu) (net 13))
 (segment (start 107.359001 104.349999) (end 42.375001 104.349999) (width 0.5) (layer F.Cu) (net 13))
 (segment (start 42.375001 104.349999) (end 41.4 105.325) (width 0.5) (layer F.Cu) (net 13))
 (segment (start 41.4 105.325) (end 40.35 105.325) (width 0.5) (layer F.Cu) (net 13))
 (segment (start 117.983 89.8525) (end 117.983 93.091) (width 0.5) (layer B.Cu) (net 13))
 (segment (start 117.983 93.091) (end 118.3005 93.4085) (width 0.5) (layer B.Cu) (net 13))
 (via (at 118.3005 93.4085) (size 0.6) (drill 0.4) (layers F.Cu B.Cu) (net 13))
 (segment (start 109.9185 89.027) (end 117.1575 89.027) (width 0.5) (layer F.Cu) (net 13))
 (via (at 117.983 89.8525) (size 0.6) (drill 0.4) (layers F.Cu B.Cu) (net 13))
 (segment (start 117.1575 89.027) (end 117.983 89.8525) (width 0.5) (layer F.Cu) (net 13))
 (segment (start 32.55 105.325) (end 32.55 104.5) (width 0.5) (layer F.Cu) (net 12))
 (segment (start 32.55 104.5) (end 45.483 91.567) (width 0.5) (layer F.Cu) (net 12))
 (segment (start 106.176419 91.567) (end 107.3785 91.567) (width 0.5) (layer F.Cu) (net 12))
 (segment (start 45.483 91.567) (end 106.176419 91.567) (width 0.5) (layer F.Cu) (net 12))
 (segment (start 117.856 108.458) (end 79.533 108.458) (width 0.5) (layer F.Cu) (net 11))
 (segment (start 79.533 108.458) (end 76.4 105.325) (width 0.5) (layer F.Cu) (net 11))
 (segment (start 76.4 105.325) (end 75.35 105.325) (width 0.5) (layer F.Cu) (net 11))
 (segment (start 118.745 107.569) (end 117.856 108.458) (width 0.5) (layer F.Cu) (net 11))
 (segment (start 118.745 98.975002) (end 118.745 107.569) (width 0.5) (layer F.Cu) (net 11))
 (segment (start 119.253 91.8845) (end 119.253 98.467002) (width 0.5) (layer F.Cu) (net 11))
 (segment (start 119.253 98.467002) (end 118.745 98.975002) (width 0.5) (layer F.Cu) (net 11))
 (segment (start 118.9355 91.567) (end 119.253 91.8845) (width 0.5) (layer F.Cu) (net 11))
 (segment (start 109.9185 91.567) (end 118.9355 91.567) (width 0.5) (layer F.Cu) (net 11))
 (via (at 109.9185 91.567) (size 0.6) (drill 0.4) (layers F.Cu B.Cu) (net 11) (status 30))
 (segment (start 63.373 102.489) (end 71.755 94.107) (width 0.5) (layer F.Cu) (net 10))
 (segment (start 71.755 94.107) (end 107.3785 94.107) (width 0.5) (layer F.Cu) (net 10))
 (segment (start 63.373 106.001736) (end 63.373 102.489) (width 0.5) (layer B.Cu) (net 10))
 (via (at 63.373 102.489) (size 0.6) (drill 0.4) (layers F.Cu B.Cu) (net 10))
 (segment (start 63.373 106.426) (end 63.373 106.001736) (width 0.5) (layer B.Cu) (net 10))
 (segment (start 67.55 105.325) (end 64.474 105.325) (width 0.5) (layer F.Cu) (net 10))
 (segment (start 64.474 105.325) (end 63.373 106.426) (width 0.5) (layer F.Cu) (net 10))
 (via (at 63.373 106.426) (size 0.6) (drill 0.4) (layers F.Cu B.Cu) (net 10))
 (segment (start 114.9985 94.1705) (end 109.982 94.1705) (width 0.5) (layer F.Cu) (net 9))
 (segment (start 109.982 94.1705) (end 109.9185 94.107) (width 0.5) (layer F.Cu) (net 9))
 (segment (start 116.0145 94.2975) (end 115.1255 94.2975) (width 0.5) (layer B.Cu) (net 9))
 (segment (start 115.1255 94.2975) (end 114.9985 94.1705) (width 0.5) (layer B.Cu) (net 9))
 (via (at 114.9985 94.1705) (size 0.6) (drill 0.4) (layers F.Cu B.Cu) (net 9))
 (via (at 116.0145 94.2975) (size 0.6) (drill 0.4) (layers F.Cu B.Cu) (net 9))
 (segment (start 116.0145 97.0915) (end 116.0145 94.2975) (width 0.5) (layer B.Cu) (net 9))
 (segment (start 116.0145 98.8355) (end 116.0145 97.0915) (width 0.5) (layer F.Cu) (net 9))
 (via (at 116.0145 97.0915) (size 0.6) (drill 0.4) (layers F.Cu B.Cu) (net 9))
 (segment (start 110.35 105.325) (end 110.35 104.5) (width 0.5) (layer F.Cu) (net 9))
 (segment (start 110.35 104.5) (end 116.0145 98.8355) (width 0.5) (layer F.Cu) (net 9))
 (segment (start 100.584 102.87) (end 106.807 96.647) (width 0.5) (layer F.Cu) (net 8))
 (segment (start 106.807 96.647) (end 107.3785 96.647) (width 0.5) (layer F.Cu) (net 8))
 (segment (start 100.203 104.8385) (end 100.203 103.251) (width 0.5) (layer B.Cu) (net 8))
 (segment (start 100.203 103.251) (end 100.584 102.87) (width 0.5) (layer B.Cu) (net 8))
 (via (at 100.584 102.87) (size 0.6) (drill 0.4) (layers F.Cu B.Cu) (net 8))
 (segment (start 99.568 105.4735) (end 100.203 104.8385) (width 0.5) (layer B.Cu) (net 8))
 (segment (start 102.55 105.325) (end 99.7165 105.325) (width 0.5) (layer F.Cu) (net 8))
 (segment (start 99.7165 105.325) (end 99.568 105.4735) (width 0.5) (layer F.Cu) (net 8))
 (via (at 99.568 105.4735) (size 0.6) (drill 0.4) (layers F.Cu B.Cu) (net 8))
 (segment (start 110.35 36.15) (end 112.2365 38.0365) (width 0.5) (layer F.Cu) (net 19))
 (segment (start 112.2365 38.0365) (end 112.450011 38.250011) (width 0.5) (layer F.Cu) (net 19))
 (segment (start 115.697 79.9465) (end 115.697 41.497) (width 0.5) (layer F.Cu) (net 19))
 (segment (start 115.697 41.497) (end 112.2365 38.0365) (width 0.5) (layer F.Cu) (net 19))
 (segment (start 114.3 81.3435) (end 115.697 79.9465) (width 0.5) (layer F.Cu) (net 19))
 (segment (start 111.184081 81.3435) (end 114.3 81.3435) (width 0.5) (layer F.Cu) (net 19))
 (segment (start 109.9185 81.407) (end 111.120581 81.407) (width 0.5) (layer F.Cu) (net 19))
 (segment (start 111.120581 81.407) (end 111.184081 81.3435) (width 0.5) (layer F.Cu) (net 19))
 (segment (start 110.35 35.325) (end 110.35 36.15) (width 0.5) (layer F.Cu) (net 19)))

